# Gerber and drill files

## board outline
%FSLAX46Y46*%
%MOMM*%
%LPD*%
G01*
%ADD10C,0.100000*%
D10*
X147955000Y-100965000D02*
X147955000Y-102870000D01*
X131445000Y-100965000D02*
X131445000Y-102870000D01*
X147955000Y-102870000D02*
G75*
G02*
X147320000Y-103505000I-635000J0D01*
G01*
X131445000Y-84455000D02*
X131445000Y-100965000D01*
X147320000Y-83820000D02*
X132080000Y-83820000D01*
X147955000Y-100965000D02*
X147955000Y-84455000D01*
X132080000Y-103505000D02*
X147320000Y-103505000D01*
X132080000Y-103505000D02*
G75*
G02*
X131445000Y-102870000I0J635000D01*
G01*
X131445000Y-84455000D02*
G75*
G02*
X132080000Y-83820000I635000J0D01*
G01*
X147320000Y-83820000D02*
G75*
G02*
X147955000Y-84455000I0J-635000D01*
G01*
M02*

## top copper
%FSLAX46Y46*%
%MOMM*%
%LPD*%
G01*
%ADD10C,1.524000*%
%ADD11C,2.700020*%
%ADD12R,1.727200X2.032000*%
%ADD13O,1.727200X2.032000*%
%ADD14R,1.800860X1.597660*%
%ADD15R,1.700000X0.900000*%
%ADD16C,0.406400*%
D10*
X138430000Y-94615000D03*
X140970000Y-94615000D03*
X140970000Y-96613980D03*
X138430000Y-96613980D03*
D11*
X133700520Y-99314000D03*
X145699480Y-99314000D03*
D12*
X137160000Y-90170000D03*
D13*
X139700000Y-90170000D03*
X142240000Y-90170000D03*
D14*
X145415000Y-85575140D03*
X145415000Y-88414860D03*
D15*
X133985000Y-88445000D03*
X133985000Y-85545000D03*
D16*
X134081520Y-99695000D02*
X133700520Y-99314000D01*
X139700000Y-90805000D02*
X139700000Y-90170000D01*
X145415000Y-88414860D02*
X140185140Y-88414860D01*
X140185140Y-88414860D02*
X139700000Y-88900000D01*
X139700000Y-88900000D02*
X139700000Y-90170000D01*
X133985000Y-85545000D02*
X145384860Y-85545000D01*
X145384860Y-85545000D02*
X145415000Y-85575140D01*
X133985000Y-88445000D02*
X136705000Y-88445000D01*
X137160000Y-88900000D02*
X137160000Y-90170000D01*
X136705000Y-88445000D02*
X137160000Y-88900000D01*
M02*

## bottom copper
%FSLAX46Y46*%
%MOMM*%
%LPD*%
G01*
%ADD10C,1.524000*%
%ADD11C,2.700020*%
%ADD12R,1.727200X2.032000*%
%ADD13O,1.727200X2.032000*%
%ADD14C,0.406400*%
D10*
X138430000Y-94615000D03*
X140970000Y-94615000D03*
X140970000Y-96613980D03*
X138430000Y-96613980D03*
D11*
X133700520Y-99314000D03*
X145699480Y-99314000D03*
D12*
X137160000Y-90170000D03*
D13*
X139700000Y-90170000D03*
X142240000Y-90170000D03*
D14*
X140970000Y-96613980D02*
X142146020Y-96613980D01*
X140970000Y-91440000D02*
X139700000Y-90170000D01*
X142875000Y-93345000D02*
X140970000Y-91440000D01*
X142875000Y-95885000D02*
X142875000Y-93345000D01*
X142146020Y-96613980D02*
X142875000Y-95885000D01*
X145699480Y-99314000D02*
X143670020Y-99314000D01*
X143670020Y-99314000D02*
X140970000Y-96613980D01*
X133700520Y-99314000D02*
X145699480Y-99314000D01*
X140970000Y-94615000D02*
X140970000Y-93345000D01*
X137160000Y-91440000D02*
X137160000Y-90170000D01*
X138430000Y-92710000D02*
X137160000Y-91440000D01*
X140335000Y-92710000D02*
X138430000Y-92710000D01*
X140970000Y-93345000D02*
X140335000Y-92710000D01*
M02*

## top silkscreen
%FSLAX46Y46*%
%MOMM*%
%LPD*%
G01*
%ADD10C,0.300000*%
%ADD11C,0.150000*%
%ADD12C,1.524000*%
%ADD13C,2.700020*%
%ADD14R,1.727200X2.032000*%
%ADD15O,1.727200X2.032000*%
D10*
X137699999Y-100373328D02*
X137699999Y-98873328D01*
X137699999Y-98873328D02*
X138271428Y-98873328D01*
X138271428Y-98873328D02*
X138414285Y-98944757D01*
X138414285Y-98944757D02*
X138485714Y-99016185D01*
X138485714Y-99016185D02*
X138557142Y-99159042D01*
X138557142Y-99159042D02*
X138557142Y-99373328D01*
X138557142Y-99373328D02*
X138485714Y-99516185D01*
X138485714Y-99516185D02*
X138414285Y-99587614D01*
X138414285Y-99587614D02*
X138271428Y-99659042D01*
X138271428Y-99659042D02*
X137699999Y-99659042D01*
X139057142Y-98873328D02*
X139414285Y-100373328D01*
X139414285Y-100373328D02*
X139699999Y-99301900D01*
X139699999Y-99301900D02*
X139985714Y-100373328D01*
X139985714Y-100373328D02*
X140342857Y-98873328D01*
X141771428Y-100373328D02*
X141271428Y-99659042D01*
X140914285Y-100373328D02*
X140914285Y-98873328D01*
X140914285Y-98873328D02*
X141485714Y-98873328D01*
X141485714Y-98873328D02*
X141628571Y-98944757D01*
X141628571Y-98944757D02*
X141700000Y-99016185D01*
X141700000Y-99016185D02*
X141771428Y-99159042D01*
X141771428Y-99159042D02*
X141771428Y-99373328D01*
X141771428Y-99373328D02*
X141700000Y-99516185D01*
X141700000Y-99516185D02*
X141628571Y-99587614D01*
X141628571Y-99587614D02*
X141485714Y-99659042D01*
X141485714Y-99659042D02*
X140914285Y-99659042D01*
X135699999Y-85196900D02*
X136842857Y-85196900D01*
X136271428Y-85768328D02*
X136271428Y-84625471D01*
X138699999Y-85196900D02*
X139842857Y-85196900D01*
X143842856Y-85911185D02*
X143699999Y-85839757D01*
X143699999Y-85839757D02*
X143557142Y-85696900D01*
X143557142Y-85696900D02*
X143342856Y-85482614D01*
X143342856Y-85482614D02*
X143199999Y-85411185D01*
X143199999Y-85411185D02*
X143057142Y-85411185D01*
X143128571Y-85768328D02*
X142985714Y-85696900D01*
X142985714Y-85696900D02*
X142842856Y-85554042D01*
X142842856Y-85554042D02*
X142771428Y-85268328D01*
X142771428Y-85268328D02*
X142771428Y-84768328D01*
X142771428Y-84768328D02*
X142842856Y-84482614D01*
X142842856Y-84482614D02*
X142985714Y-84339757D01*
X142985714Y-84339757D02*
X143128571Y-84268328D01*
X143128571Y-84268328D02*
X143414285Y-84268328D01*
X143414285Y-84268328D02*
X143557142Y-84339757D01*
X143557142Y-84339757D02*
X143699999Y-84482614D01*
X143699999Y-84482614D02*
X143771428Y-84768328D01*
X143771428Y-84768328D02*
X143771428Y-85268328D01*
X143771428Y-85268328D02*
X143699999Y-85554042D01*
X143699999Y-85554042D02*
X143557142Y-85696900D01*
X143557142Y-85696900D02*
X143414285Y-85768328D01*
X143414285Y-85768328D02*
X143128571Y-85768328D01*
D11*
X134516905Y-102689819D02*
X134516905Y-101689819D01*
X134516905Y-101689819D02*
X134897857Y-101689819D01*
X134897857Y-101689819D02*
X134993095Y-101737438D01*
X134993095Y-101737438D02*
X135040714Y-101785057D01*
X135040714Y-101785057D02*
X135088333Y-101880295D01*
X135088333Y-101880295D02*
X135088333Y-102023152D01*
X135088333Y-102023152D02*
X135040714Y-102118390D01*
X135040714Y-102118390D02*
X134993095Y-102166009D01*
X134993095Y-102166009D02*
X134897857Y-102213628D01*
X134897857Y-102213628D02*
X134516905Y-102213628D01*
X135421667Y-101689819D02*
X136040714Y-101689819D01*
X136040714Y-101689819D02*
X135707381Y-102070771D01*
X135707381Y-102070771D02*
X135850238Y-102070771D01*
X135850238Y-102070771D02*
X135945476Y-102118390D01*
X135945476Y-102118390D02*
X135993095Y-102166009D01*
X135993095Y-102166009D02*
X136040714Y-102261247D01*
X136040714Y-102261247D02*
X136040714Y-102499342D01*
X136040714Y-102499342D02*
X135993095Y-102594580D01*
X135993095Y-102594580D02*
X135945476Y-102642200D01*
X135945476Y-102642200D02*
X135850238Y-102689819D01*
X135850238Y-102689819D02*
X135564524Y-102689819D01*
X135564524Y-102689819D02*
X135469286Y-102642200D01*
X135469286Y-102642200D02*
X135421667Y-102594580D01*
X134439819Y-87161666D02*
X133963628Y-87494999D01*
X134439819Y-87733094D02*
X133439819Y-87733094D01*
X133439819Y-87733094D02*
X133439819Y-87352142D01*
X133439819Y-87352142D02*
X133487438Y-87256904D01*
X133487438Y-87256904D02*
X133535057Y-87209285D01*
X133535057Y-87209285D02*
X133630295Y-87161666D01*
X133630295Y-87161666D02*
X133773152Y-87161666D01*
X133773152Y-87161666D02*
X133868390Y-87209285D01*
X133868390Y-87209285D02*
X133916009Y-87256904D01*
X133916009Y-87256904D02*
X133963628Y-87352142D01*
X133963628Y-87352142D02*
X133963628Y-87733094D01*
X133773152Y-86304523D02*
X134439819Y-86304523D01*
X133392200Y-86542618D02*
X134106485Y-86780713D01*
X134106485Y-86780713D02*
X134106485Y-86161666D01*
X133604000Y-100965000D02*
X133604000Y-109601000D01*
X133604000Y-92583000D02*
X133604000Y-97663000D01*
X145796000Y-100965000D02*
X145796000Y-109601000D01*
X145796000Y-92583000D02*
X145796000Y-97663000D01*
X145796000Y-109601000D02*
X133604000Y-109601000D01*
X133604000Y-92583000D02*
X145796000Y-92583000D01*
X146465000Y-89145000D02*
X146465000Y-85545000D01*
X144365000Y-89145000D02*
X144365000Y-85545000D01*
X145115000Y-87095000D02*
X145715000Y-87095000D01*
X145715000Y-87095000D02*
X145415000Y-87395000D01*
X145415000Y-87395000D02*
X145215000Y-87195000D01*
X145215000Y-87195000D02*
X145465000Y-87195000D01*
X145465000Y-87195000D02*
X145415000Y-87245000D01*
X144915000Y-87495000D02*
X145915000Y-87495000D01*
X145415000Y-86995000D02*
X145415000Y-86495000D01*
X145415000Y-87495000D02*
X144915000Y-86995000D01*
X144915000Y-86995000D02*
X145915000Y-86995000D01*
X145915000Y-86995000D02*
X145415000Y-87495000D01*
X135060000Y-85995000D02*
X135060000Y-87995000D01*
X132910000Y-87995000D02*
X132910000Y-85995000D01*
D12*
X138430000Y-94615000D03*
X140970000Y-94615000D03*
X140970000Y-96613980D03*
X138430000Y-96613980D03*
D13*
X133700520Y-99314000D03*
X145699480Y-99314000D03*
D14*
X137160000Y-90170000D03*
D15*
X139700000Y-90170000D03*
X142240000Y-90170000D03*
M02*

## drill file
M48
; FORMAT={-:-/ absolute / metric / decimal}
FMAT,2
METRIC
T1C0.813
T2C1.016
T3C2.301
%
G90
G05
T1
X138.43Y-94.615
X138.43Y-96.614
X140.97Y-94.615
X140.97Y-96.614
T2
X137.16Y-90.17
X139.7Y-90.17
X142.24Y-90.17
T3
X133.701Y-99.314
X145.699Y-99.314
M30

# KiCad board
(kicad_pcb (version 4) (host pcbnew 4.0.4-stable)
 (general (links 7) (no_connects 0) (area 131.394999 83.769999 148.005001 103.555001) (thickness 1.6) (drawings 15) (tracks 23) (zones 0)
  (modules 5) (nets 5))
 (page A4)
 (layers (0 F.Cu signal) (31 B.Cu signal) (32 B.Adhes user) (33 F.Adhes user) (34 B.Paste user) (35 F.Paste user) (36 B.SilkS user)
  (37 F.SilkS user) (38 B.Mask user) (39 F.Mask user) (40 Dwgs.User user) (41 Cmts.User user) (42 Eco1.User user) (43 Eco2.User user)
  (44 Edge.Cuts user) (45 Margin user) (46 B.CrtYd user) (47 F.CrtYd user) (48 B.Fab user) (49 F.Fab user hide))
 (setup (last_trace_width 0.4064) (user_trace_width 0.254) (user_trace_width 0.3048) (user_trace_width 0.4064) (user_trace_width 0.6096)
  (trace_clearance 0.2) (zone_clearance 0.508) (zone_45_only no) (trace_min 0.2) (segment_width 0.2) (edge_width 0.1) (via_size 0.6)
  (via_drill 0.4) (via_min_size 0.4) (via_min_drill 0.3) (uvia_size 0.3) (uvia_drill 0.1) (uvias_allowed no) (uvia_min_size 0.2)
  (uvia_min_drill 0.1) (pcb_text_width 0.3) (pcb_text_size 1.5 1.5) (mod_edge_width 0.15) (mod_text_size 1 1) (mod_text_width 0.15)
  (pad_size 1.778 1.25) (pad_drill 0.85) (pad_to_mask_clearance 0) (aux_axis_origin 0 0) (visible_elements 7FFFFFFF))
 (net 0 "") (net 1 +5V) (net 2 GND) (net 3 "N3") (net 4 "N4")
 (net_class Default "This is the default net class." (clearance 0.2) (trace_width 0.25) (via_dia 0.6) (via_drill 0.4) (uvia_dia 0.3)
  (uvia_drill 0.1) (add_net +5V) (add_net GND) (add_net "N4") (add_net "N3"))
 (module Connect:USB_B (layer F.Cu) (at 140.97 94.615 270)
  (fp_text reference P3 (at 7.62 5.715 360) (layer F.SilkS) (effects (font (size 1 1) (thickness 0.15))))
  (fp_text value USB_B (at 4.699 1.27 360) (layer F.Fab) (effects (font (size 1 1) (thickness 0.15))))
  (fp_line (start 6.35 7.366) (end 14.986 7.366) (layer F.SilkS) (width 0.15))
  (fp_line (start -2.032 7.366) (end 3.048 7.366) (layer F.SilkS) (width 0.15))
  (fp_line (start 6.35 -4.826) (end 14.986 -4.826) (layer F.SilkS) (width 0.15))
  (fp_line (start -2.032 -4.826) (end 3.048 -4.826) (layer F.SilkS) (width 0.15))
  (fp_line (start 14.986 -4.826) (end 14.986 7.366) (layer F.SilkS) (width 0.15))
  (fp_line (start -2.032 7.366) (end -2.032 -4.826) (layer F.SilkS) (width 0.15))
  (pad 2 thru_hole circle (at 0 2.54 180) (size 1.524 1.524) (drill 0.8128) (layers *.Cu *.Mask F.SilkS))
  (pad 1 thru_hole circle (at 0 0 180) (size 1.524 1.524) (drill 0.8128) (layers *.Cu *.Mask F.SilkS) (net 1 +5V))
  (pad 4 thru_hole circle (at 1.99898 0 180) (size 1.524 1.524) (drill 0.8128) (layers *.Cu *.Mask F.SilkS) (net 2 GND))
  (pad 3 thru_hole circle (at 1.99898 2.54 180) (size 1.524 1.524) (drill 0.8128) (layers *.Cu *.Mask F.SilkS))
  (pad 5 thru_hole circle (at 4.699 7.26948 180) (size 2.70002 2.70002) (drill 2.30124) (layers *.Cu *.Mask F.SilkS) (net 2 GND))
  (pad 5 thru_hole circle (at 4.699 -4.72948 180) (size 2.70002 2.70002) (drill 2.30124) (layers *.Cu *.Mask F.SilkS) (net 2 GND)))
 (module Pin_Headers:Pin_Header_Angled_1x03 (layer F.Cu) (at 137.16 90.17 90)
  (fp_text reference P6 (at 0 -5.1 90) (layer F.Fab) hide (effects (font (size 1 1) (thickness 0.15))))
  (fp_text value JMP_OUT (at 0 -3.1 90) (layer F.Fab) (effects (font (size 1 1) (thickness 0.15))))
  (pad 1 thru_hole rect (at 0 0 90) (size 2.032 1.7272) (drill 1.016) (layers *.Cu *.Mask F.SilkS) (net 1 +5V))
  (pad 2 thru_hole oval (at 0 2.54 90) (size 2.032 1.7272) (drill 1.016) (layers *.Cu *.Mask F.SilkS) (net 2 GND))
  (pad 3 thru_hole oval (at 0 5.08 90) (size 2.032 1.7272) (drill 1.016) (layers *.Cu *.Mask F.SilkS) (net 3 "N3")))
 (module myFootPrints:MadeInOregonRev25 (layer F.Cu) (at 139.7 100.33)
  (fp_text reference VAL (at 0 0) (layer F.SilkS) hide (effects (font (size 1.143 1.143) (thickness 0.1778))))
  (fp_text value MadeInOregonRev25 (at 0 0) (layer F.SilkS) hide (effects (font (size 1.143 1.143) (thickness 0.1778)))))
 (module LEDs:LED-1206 (layer F.Cu) (at 145.415 86.995 90)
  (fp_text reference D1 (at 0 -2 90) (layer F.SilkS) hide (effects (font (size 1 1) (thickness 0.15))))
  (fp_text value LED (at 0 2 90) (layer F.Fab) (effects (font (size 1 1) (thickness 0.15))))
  (fp_line (start -2.15 1.05) (end 1.45 1.05) (layer F.SilkS) (width 0.15))
  (fp_line (start -2.15 -1.05) (end 1.45 -1.05) (layer F.SilkS) (width 0.15))
  (fp_line (start -0.1 -0.3) (end -0.1 0.3) (layer F.SilkS) (width 0.15))
  (fp_line (start -0.1 0.3) (end -0.4 0) (layer F.SilkS) (width 0.15))
  (fp_line (start -0.4 0) (end -0.2 -0.2) (layer F.SilkS) (width 0.15))
  (fp_line (start -0.2 -0.2) (end -0.2 0.05) (layer F.SilkS) (width 0.15))
  (fp_line (start -0.2 0.05) (end -0.25 0) (layer F.SilkS) (width 0.15))
  (fp_line (start -0.5 -0.5) (end -0.5 0.5) (layer F.SilkS) (width 0.15))
  (fp_line (start 0 0) (end 0.5 0) (layer F.SilkS) (width 0.15))
  (fp_line (start -0.5 0) (end 0 -0.5) (layer F.SilkS) (width 0.15))
  (fp_line (start 0 -0.5) (end 0 0.5) (layer F.SilkS) (width 0.15))
  (fp_line (start 0 0.5) (end -0.5 0) (layer F.SilkS) (width 0.15))
  (pad 2 smd rect (at 1.41986 0 270) (size 1.59766 1.80086) (layers F.Cu F.Paste F.Mask) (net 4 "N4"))
  (pad 1 smd rect (at -1.41986 0 270) (size 1.59766 1.80086) (layers F.Cu F.Paste F.Mask) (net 2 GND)))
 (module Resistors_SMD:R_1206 (layer F.Cu) (at 133.985 86.995 90)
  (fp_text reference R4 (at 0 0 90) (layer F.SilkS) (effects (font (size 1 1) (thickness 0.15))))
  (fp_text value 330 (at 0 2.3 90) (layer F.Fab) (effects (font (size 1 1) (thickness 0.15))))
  (fp_line (start 1 1.075) (end -1 1.075) (layer F.SilkS) (width 0.15))
  (fp_line (start -1 -1.075) (end 1 -1.075) (layer F.SilkS) (width 0.15))
  (pad 1 smd rect (at -1.45 0 90) (size 0.9 1.7) (layers F.Cu F.Paste F.Mask) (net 1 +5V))
  (pad 2 smd rect (at 1.45 0 90) (size 0.9 1.7) (layers F.Cu F.Paste F.Mask) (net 4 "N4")))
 (gr_line (start 147.955 100.965) (end 147.955 102.87) (angle 90) (layer Edge.Cuts) (width 0.1))
 (gr_line (start 131.445 100.965) (end 131.445 102.87) (angle 90) (layer Edge.Cuts) (width 0.1))
 (gr_arc (start 147.32 102.87) (end 147.955 102.87) (angle 90) (layer Edge.Cuts) (width 0.1))
 (gr_line (start 131.445 84.455) (end 131.445 100.965) (angle 90) (layer Edge.Cuts) (width 0.1))
 (gr_line (start 147.32 83.82) (end 132.08 83.82) (angle 90) (layer Edge.Cuts) (width 0.1))
 (gr_line (start 147.955 100.965) (end 147.955 84.455) (angle 90) (layer Edge.Cuts) (width 0.1))
 (gr_line (start 132.08 103.505) (end 147.32 103.505) (angle 90) (layer Edge.Cuts) (width 0.1))
 (gr_arc (start 132.08 102.87) (end 132.08 103.505) (angle 90) (layer Edge.Cuts) (width 0.1))
 (gr_arc (start 132.08 84.455) (end 131.445 84.455) (angle 90) (layer Edge.Cuts) (width 0.1))
 (gr_arc (start 147.32 84.455) (end 147.32 83.82) (angle 90) (layer Edge.Cuts) (width 0.1))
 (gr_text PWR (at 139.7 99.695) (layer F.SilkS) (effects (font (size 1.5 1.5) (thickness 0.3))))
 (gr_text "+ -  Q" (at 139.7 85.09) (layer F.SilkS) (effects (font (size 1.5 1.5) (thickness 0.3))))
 (segment (start 140.97 96.61398) (end 142.14602 96.61398) (width 0.4064) (layer B.Cu) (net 2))
 (segment (start 140.97 91.44) (end 139.7 90.17) (width 0.4064) (layer B.Cu) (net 2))
 (segment (start 142.875 93.345) (end 140.97 91.44) (width 0.4064) (layer B.Cu) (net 2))
 (segment (start 142.875 95.885) (end 142.875 93.345) (width 0.4064) (layer B.Cu) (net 2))
 (segment (start 142.14602 96.61398) (end 142.875 95.885) (width 0.4064) (layer B.Cu) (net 2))
 (segment (start 145.69948 99.314) (end 143.67002 99.314) (width 0.4064) (layer B.Cu) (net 2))
 (segment (start 143.67002 99.314) (end 140.97 96.61398) (width 0.4064) (layer B.Cu) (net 2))
 (segment (start 133.70052 99.314) (end 145.69948 99.314) (width 0.4064) (layer B.Cu) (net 2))
 (segment (start 134.08152 99.695) (end 133.70052 99.314) (width 0.4064) (layer F.Cu) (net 2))
 (segment (start 139.7 90.805) (end 139.7 90.17) (width 0.4064) (layer F.Cu) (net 2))
 (segment (start 145.415 88.41486) (end 140.18514 88.41486) (width 0.4064) (layer F.Cu) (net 2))
 (segment (start 140.18514 88.41486) (end 139.7 88.9) (width 0.4064) (layer F.Cu) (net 2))
 (segment (start 139.7 88.9) (end 139.7 90.17) (width 0.4064) (layer F.Cu) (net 2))
 (segment (start 133.985 85.545) (end 145.38486 85.545) (width 0.4064) (layer F.Cu) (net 4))
 (segment (start 145.38486 85.545) (end 145.415 85.57514) (width 0.4064) (layer F.Cu) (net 4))
 (segment (start 140.97 94.615) (end 140.97 93.345) (width 0.4064) (layer B.Cu) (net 1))
 (segment (start 137.16 91.44) (end 137.16 90.17) (width 0.4064) (layer B.Cu) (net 1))
 (segment (start 138.43 92.71) (end 137.16 91.44) (width 0.4064) (layer B.Cu) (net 1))
 (segment (start 140.335 92.71) (end 138.43 92.71) (width 0.4064) (layer B.Cu) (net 1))
 (segment (start 140.97 93.345) (end 140.335 92.71) (width 0.4064) (layer B.Cu) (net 1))
 (segment (start 133.985 88.445) (end 136.705 88.445) (width 0.4064) (layer F.Cu) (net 1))
 (segment (start 137.16 88.9) (end 137.16 90.17) (width 0.4064) (layer F.Cu) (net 1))
 (segment (start 136.705 88.445) (end 137.16 88.9) (width 0.4064) (layer F.Cu) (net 1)))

